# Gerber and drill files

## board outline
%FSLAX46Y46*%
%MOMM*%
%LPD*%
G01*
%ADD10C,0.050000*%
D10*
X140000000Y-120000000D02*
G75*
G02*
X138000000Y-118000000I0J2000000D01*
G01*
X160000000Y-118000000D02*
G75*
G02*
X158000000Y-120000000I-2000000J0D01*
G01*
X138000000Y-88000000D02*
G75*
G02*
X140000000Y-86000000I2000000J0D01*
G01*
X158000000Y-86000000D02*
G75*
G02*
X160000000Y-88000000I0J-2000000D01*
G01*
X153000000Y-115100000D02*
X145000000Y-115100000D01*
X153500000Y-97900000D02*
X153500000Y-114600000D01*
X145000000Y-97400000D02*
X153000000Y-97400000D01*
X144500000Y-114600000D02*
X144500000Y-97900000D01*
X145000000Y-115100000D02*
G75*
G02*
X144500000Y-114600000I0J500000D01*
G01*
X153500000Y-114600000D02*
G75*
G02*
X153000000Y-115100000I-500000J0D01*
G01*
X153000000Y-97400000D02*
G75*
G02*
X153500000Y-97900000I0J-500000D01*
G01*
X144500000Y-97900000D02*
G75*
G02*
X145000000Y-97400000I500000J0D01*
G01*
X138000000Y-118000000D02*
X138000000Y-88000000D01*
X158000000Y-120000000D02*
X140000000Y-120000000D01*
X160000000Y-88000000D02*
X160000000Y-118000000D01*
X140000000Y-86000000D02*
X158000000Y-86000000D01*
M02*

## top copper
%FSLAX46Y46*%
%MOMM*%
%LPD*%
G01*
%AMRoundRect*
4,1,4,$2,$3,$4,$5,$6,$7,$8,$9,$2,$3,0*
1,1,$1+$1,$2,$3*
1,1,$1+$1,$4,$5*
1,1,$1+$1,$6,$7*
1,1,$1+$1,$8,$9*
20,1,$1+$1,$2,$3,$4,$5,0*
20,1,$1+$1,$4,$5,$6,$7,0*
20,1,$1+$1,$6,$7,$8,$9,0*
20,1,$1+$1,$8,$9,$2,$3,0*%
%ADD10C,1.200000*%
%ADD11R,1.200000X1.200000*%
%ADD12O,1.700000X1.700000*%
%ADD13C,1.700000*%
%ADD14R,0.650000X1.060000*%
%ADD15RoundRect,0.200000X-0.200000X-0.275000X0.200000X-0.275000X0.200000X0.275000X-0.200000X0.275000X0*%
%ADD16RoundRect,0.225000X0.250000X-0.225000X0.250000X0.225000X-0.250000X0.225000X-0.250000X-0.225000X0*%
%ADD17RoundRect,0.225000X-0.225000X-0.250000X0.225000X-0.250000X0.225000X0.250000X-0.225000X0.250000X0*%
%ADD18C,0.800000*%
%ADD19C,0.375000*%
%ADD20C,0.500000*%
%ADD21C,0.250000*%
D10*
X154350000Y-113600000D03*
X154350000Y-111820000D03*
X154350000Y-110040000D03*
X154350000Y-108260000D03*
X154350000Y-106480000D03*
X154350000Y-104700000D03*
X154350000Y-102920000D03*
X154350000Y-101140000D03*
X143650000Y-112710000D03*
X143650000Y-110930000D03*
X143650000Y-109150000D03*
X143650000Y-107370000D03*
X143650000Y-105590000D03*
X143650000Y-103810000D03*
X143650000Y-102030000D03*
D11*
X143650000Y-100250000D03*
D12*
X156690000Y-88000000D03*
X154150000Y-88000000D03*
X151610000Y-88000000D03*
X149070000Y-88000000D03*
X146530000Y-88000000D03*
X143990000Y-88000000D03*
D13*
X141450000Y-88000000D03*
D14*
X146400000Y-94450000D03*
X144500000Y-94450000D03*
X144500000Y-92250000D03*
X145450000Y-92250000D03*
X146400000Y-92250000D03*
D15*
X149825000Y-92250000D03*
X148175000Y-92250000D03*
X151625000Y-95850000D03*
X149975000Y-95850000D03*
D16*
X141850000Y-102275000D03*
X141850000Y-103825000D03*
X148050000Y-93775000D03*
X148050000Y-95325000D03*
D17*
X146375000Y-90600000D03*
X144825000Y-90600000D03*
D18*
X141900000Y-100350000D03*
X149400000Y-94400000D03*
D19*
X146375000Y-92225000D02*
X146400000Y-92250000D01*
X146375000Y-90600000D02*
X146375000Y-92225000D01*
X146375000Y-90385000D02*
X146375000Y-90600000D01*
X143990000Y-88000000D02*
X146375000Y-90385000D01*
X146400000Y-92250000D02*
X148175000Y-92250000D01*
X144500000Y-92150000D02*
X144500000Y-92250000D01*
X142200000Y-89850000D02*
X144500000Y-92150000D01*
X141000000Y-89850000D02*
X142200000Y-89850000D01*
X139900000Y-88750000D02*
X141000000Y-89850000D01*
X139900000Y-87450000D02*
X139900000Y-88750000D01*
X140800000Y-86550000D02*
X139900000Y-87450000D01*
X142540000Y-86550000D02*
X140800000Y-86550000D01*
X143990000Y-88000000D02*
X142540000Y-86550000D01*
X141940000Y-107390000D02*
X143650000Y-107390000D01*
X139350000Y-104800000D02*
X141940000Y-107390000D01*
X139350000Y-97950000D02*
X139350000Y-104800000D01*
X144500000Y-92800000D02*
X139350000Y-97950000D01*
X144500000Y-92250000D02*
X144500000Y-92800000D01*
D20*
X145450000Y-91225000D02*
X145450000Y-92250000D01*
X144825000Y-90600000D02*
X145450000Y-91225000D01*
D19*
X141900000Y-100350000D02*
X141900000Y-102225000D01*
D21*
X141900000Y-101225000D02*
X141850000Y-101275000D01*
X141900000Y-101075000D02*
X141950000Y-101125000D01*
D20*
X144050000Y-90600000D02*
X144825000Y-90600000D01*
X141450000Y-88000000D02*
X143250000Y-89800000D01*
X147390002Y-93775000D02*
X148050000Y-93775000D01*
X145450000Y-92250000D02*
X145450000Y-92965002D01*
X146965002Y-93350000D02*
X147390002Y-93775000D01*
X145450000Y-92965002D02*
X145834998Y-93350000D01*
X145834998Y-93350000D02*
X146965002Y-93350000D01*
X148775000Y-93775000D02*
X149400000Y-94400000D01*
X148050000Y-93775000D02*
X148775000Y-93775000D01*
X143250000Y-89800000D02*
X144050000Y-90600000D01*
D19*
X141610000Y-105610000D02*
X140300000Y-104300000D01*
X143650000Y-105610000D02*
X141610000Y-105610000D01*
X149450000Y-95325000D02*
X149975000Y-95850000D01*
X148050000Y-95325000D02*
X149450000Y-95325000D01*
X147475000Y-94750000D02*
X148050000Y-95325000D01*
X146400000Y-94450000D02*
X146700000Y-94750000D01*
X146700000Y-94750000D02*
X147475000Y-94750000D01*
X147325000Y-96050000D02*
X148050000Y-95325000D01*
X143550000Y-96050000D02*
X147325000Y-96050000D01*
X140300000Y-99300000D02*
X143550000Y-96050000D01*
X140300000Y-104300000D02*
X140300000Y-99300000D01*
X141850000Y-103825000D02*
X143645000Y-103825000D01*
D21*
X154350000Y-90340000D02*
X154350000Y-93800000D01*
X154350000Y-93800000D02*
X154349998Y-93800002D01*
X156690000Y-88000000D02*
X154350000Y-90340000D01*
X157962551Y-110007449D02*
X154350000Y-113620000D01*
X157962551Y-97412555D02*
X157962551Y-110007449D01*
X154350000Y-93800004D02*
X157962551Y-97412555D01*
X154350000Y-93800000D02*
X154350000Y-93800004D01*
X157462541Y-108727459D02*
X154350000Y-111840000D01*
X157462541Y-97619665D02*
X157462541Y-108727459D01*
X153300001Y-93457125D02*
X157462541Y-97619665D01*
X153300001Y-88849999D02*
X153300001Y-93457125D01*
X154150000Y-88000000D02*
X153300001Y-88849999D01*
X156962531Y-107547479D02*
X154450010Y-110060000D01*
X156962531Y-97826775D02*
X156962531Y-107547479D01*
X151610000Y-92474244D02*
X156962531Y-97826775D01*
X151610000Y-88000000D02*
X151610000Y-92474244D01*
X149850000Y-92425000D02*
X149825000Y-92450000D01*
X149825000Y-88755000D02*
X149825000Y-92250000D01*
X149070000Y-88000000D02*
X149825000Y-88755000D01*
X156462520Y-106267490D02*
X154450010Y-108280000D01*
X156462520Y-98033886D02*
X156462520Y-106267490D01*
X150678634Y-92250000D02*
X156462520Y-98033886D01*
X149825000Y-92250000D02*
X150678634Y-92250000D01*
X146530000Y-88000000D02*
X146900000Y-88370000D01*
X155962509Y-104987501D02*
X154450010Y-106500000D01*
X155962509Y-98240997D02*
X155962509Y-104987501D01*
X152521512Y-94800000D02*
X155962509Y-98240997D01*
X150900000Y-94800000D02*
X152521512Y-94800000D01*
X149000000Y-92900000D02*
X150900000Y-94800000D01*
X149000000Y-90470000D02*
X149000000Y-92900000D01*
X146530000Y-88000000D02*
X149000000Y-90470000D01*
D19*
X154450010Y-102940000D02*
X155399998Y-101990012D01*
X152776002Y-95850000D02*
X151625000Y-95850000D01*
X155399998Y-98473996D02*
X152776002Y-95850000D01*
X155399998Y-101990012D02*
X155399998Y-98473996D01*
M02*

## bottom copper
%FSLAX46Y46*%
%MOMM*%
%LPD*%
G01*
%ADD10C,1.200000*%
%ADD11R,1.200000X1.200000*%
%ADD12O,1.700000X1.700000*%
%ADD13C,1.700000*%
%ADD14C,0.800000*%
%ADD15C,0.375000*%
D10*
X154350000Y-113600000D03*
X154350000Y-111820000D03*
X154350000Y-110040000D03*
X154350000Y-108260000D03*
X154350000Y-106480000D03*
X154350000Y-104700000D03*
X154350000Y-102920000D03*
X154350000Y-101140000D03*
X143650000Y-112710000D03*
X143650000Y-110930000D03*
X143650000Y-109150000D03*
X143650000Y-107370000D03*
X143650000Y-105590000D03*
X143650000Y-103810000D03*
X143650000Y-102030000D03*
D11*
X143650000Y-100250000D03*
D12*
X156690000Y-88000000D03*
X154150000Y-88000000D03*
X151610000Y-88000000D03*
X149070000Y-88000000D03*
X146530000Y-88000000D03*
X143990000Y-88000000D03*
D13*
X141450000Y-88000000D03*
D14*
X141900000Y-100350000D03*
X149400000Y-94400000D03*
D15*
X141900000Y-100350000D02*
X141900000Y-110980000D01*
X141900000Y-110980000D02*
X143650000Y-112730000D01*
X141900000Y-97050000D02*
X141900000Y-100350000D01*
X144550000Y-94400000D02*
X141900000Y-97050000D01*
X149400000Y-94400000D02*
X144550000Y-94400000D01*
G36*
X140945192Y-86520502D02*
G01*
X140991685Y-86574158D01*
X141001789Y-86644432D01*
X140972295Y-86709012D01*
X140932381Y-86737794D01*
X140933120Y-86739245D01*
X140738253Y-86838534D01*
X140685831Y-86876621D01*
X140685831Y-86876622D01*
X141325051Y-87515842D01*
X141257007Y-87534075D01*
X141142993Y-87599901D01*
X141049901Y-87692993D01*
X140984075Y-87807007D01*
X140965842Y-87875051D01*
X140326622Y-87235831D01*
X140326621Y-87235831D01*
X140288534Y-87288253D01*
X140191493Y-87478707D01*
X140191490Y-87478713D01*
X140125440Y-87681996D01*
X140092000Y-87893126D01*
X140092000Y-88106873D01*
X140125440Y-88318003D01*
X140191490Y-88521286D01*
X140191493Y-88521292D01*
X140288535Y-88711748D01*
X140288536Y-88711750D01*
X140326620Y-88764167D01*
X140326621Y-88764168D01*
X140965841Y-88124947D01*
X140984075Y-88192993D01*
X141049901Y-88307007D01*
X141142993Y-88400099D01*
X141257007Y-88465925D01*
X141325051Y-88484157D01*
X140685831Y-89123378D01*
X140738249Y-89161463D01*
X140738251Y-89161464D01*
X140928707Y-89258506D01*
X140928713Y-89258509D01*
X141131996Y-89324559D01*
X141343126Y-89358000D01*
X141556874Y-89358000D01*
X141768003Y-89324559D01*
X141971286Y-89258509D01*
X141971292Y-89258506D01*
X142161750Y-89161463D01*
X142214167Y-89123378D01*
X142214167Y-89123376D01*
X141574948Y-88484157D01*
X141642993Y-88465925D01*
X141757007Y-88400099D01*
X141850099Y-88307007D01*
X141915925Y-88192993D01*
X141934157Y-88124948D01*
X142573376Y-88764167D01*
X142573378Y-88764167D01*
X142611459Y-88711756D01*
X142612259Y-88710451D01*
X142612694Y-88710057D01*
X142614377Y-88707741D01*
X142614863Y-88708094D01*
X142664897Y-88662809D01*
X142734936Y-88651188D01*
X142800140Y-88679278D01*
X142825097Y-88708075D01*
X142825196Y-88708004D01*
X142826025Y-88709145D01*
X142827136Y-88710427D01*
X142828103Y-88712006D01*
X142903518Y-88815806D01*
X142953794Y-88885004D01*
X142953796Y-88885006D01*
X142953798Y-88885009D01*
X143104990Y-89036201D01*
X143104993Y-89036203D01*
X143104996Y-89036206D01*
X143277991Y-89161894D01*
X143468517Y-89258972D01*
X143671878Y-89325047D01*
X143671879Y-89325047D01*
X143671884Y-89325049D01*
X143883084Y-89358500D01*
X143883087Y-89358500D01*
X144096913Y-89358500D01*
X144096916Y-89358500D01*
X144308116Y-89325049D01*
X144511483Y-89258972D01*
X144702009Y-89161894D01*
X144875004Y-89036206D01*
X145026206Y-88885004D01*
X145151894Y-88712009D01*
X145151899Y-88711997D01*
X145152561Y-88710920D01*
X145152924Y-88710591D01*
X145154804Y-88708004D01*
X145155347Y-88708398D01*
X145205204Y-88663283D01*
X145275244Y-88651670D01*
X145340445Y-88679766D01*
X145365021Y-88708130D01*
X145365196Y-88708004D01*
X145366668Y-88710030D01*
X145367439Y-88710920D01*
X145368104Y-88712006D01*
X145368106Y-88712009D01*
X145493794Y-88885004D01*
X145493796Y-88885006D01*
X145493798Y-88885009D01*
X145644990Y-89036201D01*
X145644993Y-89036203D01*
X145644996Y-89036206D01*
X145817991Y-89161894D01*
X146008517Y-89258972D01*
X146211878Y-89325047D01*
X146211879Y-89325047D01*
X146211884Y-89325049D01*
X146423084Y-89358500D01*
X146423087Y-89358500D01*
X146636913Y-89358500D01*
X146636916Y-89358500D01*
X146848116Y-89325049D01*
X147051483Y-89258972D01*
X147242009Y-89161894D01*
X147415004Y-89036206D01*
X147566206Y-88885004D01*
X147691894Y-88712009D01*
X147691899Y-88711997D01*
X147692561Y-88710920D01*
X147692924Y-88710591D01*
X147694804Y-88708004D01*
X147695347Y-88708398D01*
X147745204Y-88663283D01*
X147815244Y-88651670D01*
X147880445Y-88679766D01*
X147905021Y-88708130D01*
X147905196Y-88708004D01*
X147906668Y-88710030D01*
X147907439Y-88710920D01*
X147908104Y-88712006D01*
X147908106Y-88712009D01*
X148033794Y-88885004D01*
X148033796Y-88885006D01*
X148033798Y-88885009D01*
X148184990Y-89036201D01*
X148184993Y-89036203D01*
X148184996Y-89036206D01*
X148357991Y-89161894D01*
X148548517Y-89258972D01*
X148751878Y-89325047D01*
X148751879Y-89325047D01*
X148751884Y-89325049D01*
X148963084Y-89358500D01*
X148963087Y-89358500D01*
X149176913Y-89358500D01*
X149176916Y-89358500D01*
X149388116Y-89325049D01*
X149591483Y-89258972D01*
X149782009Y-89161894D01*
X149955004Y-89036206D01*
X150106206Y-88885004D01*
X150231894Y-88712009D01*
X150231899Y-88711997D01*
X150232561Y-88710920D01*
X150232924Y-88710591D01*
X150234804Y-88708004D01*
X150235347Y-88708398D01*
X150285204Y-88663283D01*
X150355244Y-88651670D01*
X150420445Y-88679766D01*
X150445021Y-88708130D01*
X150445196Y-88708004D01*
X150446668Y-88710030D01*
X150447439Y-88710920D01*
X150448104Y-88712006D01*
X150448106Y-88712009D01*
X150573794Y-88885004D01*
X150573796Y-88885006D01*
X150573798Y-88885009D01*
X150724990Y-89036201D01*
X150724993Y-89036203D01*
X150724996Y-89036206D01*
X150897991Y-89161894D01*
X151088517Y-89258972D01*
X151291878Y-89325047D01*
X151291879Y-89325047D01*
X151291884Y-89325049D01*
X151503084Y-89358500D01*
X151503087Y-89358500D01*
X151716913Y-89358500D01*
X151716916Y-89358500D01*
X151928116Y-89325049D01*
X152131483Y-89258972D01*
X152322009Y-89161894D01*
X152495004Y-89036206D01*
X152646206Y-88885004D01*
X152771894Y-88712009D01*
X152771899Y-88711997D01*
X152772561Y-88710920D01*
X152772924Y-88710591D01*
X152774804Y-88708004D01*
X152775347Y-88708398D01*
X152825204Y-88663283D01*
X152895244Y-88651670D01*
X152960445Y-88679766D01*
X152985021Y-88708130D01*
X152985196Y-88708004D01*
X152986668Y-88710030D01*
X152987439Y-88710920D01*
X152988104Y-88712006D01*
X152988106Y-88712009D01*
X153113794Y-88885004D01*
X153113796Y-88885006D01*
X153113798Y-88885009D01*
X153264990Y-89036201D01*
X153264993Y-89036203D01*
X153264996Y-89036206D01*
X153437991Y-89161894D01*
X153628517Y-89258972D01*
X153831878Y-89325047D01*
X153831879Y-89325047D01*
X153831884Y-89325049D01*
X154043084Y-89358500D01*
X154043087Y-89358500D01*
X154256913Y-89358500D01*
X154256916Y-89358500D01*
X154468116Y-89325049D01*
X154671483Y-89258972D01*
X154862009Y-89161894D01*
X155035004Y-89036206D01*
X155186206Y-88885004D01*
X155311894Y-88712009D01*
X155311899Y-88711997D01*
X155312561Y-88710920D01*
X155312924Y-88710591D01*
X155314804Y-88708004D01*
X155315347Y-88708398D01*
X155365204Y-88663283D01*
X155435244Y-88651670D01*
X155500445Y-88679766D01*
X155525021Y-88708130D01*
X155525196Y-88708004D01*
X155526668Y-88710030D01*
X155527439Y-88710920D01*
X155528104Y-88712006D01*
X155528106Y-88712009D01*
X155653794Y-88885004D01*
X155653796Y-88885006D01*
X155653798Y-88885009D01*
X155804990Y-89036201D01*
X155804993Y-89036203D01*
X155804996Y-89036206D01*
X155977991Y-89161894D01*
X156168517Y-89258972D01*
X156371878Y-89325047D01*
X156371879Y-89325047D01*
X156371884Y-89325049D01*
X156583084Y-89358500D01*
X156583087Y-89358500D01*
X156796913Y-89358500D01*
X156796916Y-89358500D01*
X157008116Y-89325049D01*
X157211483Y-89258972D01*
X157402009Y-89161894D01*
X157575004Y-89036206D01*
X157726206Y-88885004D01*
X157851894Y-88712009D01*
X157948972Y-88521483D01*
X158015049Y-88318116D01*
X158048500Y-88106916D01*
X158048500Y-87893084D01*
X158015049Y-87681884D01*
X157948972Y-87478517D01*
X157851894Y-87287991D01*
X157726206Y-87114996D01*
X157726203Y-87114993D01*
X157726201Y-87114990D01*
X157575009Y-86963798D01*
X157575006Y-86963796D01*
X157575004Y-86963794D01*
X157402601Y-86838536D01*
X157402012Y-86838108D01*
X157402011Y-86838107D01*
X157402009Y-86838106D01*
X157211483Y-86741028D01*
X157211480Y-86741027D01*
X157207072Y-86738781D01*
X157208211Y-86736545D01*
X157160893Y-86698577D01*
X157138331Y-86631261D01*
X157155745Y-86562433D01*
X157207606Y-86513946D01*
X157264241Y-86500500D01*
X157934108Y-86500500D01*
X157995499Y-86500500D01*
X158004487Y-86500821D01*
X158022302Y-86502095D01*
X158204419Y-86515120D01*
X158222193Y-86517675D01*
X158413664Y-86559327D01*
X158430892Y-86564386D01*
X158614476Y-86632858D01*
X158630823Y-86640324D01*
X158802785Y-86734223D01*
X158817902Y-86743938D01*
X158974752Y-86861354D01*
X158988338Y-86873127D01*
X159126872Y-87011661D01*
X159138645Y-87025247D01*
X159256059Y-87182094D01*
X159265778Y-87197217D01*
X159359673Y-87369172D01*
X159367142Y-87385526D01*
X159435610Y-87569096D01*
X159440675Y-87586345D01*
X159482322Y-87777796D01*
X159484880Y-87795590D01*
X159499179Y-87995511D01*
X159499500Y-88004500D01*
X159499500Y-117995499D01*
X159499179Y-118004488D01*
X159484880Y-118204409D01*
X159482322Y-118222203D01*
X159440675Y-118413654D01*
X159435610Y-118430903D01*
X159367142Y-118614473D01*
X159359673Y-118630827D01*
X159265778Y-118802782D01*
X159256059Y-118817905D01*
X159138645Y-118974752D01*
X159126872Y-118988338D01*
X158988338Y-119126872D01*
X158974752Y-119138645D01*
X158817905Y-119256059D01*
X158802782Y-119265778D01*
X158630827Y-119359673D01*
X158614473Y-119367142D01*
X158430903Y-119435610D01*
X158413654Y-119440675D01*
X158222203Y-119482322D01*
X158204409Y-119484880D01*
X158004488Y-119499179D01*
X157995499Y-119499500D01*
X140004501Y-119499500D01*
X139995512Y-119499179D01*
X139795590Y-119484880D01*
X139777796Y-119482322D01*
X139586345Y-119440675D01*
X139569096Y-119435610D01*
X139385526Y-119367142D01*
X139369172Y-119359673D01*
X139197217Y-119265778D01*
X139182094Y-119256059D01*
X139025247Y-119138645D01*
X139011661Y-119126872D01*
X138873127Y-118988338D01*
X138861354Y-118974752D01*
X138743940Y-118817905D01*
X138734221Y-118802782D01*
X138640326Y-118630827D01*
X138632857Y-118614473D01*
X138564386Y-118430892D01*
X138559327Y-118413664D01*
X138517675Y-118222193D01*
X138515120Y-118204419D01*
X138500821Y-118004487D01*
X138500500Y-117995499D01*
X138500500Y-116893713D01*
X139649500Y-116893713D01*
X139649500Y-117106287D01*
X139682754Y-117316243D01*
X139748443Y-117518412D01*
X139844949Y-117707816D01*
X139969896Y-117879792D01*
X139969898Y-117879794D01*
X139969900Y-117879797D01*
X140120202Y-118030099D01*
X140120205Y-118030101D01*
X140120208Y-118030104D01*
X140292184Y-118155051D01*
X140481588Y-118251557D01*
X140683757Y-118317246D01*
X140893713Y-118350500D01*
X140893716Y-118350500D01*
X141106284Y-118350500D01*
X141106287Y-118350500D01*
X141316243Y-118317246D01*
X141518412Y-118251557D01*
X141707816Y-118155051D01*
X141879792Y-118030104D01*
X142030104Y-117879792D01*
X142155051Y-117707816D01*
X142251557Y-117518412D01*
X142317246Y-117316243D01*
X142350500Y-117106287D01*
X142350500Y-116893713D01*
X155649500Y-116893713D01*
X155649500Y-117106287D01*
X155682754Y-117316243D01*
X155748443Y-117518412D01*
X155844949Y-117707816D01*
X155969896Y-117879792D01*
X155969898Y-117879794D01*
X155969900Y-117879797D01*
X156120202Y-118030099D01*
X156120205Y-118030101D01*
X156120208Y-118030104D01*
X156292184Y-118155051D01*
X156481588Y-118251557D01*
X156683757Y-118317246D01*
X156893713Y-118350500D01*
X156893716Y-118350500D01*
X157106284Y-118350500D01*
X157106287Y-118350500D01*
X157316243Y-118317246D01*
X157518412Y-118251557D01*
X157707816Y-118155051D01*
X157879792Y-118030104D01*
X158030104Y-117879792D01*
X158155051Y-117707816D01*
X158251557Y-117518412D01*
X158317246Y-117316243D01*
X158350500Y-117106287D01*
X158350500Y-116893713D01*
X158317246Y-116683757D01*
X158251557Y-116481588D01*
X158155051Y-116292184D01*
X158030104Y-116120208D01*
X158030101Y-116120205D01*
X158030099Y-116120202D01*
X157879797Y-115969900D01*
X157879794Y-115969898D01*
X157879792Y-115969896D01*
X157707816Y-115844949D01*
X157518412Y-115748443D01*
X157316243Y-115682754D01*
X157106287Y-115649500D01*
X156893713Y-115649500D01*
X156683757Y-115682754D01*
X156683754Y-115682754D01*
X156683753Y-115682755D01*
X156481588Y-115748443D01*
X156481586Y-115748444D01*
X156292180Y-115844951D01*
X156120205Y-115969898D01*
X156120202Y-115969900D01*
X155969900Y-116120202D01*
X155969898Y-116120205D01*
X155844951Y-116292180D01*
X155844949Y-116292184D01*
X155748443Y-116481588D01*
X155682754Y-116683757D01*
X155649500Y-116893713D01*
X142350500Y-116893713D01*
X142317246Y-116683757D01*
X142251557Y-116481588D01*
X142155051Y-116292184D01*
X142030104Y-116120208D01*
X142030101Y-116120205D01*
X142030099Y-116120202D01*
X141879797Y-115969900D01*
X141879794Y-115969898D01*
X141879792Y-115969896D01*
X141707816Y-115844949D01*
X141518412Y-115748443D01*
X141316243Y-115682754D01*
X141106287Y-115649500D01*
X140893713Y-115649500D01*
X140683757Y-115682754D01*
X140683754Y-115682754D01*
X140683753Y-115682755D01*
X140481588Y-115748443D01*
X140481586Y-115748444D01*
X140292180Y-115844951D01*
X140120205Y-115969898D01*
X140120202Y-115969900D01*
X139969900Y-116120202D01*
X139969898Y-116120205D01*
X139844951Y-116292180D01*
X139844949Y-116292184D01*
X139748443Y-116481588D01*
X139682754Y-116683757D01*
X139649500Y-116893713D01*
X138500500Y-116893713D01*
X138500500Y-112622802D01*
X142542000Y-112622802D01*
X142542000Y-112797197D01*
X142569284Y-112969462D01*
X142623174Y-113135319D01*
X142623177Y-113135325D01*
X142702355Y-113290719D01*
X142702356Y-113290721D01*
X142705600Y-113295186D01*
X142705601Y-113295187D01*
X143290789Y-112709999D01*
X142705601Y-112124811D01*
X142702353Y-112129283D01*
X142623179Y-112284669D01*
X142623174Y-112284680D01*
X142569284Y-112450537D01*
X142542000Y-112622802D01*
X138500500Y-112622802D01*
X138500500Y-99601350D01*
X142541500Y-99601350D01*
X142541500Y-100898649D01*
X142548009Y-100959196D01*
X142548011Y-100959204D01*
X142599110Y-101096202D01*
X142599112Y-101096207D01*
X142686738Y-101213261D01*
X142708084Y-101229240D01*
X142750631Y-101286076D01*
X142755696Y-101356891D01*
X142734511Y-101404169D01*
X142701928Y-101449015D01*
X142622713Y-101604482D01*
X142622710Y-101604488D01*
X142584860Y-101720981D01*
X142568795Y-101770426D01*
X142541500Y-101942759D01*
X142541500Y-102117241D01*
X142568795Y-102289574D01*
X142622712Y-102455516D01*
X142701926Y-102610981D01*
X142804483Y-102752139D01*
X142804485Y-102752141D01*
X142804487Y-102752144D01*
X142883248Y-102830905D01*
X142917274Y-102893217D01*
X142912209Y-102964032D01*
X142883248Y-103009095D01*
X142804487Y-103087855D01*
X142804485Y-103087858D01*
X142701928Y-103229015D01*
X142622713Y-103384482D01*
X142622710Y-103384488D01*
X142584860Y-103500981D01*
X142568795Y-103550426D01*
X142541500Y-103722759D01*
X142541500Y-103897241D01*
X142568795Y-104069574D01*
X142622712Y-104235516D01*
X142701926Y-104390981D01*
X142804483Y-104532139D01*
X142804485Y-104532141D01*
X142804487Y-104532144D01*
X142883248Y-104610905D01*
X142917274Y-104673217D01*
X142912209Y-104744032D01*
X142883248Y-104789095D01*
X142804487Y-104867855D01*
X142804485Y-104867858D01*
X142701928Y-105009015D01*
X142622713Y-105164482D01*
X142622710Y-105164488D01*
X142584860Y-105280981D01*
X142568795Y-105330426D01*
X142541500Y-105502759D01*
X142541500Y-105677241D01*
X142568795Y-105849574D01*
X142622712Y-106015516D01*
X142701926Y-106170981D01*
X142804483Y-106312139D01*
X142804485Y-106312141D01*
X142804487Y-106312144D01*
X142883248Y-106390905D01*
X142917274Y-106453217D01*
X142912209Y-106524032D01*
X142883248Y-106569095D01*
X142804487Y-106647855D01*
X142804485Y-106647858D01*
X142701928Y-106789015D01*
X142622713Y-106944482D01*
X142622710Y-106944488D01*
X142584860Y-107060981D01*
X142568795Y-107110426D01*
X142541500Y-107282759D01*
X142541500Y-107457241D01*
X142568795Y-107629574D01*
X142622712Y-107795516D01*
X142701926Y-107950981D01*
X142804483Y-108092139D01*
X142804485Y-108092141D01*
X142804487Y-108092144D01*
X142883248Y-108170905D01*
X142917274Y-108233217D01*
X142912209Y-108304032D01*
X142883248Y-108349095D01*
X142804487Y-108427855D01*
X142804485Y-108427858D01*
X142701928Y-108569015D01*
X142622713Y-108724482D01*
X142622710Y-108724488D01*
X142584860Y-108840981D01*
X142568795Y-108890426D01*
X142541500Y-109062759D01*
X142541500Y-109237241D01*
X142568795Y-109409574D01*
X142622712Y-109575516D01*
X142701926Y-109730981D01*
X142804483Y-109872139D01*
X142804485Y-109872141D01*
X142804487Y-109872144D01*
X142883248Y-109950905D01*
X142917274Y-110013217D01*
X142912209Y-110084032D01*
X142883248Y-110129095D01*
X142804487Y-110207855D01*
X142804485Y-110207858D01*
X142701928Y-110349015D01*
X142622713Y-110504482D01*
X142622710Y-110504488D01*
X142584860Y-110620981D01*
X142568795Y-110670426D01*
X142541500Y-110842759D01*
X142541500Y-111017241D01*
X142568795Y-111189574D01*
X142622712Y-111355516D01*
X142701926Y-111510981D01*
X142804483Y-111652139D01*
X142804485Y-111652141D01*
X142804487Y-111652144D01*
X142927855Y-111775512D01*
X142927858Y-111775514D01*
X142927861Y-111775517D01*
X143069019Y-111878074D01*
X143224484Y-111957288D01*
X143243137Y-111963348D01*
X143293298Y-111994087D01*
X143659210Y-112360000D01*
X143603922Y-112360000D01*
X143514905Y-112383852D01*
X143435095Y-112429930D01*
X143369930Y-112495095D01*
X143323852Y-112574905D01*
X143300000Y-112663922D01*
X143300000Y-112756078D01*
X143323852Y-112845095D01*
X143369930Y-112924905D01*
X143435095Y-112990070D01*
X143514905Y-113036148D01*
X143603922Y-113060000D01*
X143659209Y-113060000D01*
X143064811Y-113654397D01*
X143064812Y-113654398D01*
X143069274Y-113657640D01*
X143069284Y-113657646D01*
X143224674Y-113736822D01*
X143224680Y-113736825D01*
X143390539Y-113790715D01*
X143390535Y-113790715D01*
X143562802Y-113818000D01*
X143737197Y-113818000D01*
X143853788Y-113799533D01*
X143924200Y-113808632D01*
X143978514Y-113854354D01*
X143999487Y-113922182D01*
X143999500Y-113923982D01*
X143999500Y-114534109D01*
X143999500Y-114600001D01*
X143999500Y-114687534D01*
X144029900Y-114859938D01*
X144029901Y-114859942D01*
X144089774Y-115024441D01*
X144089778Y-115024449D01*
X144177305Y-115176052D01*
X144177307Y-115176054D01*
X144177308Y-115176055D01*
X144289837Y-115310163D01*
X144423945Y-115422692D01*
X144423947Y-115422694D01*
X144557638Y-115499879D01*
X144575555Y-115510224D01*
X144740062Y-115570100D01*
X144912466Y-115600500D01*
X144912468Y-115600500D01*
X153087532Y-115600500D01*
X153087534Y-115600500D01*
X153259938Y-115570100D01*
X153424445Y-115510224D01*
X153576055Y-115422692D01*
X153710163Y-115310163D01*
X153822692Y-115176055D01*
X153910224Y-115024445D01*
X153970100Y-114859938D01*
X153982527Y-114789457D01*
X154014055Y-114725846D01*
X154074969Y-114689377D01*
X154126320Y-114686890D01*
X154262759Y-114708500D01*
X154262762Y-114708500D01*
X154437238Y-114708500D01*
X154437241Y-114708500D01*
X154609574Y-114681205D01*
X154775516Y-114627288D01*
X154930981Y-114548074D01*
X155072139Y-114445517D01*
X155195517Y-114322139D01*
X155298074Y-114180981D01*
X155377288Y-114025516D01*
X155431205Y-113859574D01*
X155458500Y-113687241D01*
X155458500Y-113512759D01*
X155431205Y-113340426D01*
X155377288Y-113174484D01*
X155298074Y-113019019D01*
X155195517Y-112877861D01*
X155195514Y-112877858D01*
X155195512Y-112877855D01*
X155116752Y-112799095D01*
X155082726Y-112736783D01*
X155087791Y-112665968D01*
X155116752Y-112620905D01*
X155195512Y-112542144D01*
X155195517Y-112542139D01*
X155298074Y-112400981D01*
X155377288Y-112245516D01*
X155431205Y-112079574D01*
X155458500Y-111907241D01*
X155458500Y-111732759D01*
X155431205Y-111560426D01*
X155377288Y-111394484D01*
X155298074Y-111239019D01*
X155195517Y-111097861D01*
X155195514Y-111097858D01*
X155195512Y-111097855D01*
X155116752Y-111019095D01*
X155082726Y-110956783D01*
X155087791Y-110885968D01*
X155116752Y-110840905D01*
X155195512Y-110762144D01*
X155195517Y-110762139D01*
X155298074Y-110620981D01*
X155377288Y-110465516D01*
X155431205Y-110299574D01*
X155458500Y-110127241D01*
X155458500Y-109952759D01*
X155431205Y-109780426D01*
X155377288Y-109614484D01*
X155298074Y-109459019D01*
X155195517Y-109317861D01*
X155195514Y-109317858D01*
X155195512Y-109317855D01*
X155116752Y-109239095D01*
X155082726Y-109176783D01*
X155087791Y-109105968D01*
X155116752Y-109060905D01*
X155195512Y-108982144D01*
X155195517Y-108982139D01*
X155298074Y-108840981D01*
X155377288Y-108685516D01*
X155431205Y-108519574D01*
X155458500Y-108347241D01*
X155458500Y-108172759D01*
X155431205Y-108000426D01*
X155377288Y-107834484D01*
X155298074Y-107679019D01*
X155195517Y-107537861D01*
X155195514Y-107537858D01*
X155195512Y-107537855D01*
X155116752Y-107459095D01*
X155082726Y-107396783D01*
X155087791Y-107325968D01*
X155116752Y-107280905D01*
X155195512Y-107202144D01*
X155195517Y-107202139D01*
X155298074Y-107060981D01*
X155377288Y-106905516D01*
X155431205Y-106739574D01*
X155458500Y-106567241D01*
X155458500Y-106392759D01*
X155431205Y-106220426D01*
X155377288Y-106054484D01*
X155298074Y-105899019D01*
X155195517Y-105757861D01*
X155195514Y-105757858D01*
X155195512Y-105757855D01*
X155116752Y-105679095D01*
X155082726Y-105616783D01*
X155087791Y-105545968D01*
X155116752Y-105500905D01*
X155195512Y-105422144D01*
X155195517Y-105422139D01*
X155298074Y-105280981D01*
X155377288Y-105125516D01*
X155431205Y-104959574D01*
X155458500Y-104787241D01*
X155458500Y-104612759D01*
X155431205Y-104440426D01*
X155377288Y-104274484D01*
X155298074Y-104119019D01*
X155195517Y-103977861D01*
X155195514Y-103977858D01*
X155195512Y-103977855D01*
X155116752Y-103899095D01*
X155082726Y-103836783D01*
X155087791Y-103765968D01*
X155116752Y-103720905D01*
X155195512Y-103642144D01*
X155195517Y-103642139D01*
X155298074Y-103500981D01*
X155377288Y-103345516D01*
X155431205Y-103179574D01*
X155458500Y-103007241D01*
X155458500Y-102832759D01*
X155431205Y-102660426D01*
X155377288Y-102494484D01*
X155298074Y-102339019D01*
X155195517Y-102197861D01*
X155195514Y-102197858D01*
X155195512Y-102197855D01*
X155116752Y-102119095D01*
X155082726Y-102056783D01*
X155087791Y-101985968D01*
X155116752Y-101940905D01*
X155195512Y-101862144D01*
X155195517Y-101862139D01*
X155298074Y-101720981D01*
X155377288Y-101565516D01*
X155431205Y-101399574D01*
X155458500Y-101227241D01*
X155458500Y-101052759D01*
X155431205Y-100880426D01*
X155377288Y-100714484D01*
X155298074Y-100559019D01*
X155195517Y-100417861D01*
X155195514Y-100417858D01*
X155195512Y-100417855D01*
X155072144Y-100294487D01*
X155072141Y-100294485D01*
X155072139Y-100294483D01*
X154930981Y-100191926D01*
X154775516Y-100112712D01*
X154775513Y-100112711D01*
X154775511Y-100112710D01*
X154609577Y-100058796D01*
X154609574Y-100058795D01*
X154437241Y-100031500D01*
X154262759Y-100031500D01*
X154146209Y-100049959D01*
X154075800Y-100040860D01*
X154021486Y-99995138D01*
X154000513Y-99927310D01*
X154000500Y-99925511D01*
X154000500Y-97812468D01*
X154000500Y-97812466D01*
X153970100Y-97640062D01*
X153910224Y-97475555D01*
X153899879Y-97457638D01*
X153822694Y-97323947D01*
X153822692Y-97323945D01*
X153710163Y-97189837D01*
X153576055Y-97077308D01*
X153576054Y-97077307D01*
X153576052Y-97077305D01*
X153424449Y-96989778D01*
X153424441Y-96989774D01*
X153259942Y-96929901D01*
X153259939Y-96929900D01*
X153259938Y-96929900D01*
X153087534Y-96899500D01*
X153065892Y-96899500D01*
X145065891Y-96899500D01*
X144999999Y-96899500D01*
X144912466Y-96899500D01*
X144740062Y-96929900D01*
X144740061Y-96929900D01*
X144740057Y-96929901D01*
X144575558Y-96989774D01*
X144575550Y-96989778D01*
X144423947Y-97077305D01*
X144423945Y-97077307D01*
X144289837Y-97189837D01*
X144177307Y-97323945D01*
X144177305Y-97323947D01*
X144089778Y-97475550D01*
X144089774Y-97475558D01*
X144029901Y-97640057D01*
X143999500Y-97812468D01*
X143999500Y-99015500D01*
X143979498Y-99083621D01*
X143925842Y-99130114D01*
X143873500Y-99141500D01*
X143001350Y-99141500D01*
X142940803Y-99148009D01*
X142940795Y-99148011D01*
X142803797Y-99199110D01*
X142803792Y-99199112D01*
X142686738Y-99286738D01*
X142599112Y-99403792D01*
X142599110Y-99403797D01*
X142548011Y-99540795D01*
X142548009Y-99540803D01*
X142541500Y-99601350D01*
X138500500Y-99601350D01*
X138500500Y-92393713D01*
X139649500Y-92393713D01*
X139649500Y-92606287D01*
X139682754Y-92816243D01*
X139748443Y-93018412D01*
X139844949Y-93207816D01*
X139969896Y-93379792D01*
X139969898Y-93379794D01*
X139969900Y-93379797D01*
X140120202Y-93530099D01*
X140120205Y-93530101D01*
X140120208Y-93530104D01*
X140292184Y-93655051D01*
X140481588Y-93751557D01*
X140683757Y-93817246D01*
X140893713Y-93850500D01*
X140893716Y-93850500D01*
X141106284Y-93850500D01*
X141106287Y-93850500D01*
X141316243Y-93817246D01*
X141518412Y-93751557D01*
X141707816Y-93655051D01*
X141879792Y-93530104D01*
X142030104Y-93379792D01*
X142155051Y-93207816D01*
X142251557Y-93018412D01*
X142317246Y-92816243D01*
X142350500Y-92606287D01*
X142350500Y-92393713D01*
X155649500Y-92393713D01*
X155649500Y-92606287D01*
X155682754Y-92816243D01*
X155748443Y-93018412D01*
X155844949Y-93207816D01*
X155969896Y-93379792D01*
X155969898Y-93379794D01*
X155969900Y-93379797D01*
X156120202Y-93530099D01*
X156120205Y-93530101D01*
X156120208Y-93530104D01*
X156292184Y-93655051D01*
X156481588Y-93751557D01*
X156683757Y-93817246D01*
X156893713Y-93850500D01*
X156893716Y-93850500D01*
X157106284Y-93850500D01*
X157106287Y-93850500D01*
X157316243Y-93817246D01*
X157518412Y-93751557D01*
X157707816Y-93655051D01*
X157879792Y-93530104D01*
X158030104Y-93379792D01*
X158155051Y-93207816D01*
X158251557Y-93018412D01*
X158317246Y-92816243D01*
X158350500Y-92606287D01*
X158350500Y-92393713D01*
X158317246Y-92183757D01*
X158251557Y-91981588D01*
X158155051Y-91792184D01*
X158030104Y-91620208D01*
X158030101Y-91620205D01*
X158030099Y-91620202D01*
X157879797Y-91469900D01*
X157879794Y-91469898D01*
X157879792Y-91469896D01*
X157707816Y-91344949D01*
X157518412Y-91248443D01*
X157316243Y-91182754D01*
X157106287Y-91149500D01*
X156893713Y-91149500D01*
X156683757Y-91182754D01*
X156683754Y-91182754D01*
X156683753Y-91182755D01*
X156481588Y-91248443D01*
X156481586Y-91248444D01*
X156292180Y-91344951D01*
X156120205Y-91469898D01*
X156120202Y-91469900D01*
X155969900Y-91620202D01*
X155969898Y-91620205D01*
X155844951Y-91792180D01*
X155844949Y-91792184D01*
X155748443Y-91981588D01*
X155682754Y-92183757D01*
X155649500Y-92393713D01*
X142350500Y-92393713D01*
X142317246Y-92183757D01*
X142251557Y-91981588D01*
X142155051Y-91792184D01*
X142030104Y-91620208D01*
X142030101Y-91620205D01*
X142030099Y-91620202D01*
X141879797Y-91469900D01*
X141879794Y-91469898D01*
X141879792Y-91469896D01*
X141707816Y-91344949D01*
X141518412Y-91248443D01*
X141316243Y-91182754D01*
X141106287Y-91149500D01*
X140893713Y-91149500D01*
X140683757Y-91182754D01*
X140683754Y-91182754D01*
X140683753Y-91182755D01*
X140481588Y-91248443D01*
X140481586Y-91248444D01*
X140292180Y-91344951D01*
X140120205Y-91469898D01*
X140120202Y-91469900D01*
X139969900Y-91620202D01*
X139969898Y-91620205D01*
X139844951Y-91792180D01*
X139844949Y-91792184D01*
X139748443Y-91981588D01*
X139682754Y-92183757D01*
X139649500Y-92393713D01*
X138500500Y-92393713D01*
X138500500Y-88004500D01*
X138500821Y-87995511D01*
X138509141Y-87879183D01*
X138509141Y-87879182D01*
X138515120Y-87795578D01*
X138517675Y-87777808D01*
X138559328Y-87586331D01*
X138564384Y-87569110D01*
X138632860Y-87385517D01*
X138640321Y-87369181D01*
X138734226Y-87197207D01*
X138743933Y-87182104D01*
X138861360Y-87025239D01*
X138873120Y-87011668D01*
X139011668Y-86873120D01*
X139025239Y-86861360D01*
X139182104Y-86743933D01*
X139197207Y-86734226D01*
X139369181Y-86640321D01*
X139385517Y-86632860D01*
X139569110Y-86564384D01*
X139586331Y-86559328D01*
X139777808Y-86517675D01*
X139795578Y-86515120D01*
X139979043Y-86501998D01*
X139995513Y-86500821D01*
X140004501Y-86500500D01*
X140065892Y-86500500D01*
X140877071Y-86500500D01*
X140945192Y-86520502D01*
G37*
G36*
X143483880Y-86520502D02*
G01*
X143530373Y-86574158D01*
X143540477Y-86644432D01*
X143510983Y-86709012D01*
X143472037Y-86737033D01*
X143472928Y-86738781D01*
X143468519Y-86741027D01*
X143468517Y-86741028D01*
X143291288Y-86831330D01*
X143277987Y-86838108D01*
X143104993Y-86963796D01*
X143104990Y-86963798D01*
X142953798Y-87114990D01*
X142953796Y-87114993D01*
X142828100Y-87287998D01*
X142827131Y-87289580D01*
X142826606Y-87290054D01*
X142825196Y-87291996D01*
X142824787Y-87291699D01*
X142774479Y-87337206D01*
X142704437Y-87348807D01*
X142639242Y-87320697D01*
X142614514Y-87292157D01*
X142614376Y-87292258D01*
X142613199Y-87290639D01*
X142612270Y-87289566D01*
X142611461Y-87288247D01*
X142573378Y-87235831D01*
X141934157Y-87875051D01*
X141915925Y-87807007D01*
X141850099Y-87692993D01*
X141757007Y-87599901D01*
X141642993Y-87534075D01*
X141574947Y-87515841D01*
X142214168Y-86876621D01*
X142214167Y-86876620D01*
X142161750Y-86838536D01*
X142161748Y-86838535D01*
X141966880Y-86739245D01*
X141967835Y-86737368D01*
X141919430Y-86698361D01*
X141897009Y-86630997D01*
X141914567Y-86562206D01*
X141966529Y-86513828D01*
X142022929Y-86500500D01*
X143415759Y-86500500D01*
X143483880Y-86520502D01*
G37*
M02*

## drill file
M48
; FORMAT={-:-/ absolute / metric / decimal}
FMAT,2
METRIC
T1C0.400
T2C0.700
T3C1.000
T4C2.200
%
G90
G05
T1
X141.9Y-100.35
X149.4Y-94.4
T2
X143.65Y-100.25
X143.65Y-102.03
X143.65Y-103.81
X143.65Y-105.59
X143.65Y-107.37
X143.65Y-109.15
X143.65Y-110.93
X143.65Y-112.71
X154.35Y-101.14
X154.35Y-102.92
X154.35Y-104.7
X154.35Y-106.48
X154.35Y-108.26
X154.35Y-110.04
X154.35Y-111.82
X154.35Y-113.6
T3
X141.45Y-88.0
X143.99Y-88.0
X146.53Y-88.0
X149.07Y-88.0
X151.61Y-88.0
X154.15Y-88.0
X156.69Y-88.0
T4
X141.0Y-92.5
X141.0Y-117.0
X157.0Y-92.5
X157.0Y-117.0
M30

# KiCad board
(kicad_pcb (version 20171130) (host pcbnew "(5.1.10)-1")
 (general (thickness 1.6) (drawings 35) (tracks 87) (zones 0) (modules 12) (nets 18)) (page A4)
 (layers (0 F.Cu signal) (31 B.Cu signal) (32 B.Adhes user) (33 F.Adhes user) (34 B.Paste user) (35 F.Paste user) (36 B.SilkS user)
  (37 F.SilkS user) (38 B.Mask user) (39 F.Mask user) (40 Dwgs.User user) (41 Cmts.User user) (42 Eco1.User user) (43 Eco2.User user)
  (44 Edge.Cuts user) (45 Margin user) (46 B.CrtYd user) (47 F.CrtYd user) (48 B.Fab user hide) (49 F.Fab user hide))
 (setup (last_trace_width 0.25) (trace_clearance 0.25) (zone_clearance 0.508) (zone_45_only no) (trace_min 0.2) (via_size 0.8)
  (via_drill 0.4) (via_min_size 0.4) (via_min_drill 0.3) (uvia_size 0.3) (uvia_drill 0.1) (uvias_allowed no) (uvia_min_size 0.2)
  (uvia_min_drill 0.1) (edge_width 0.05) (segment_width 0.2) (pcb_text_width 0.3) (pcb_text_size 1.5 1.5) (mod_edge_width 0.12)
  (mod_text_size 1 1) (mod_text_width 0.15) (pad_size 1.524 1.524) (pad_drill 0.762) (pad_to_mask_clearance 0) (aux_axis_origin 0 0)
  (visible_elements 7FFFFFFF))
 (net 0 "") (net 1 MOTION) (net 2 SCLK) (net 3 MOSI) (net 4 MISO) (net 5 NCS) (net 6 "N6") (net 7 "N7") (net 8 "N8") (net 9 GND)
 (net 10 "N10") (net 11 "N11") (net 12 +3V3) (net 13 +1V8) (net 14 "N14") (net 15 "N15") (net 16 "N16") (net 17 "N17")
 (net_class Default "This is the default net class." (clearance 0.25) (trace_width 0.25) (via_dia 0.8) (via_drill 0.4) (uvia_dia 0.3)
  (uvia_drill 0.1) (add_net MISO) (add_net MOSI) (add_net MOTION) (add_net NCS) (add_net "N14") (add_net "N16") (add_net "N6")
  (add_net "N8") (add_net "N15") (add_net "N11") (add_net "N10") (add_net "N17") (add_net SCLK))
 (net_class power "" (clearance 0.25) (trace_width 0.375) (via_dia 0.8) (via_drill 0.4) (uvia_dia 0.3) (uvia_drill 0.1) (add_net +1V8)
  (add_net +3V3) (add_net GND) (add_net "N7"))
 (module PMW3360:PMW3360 (layer F.Cu) (at 143.65 100.25)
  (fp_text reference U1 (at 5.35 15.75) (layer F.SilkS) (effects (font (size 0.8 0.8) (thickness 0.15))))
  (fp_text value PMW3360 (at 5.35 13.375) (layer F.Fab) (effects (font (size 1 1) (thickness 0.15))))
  (pad 9 thru_hole circle (at 10.7 13.35) (size 1.2 1.2) (drill 0.7) (layers *.Cu *.Mask) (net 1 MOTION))
  (pad 10 thru_hole circle (at 10.7 11.57) (size 1.2 1.2) (drill 0.7) (layers *.Cu *.Mask) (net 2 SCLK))
  (pad 11 thru_hole circle (at 10.7 9.79) (size 1.2 1.2) (drill 0.7) (layers *.Cu *.Mask) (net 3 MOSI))
  (pad 12 thru_hole circle (at 10.7 8.01) (size 1.2 1.2) (drill 0.7) (layers *.Cu *.Mask) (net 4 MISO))
  (pad 13 thru_hole circle (at 10.7 6.23) (size 1.2 1.2) (drill 0.7) (layers *.Cu *.Mask) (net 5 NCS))
  (pad 14 thru_hole circle (at 10.7 4.45) (size 1.2 1.2) (drill 0.7) (layers *.Cu *.Mask) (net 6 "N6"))
  (pad 15 thru_hole circle (at 10.7 2.67) (size 1.2 1.2) (drill 0.7) (layers *.Cu *.Mask) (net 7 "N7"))
  (pad 16 thru_hole circle (at 10.7 0.89) (size 1.2 1.2) (drill 0.7) (layers *.Cu *.Mask) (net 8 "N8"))
  (pad 8 thru_hole circle (at 0 12.46) (size 1.2 1.2) (drill 0.7) (layers *.Cu *.Mask) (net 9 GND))
  (pad 7 thru_hole circle (at 0 10.68) (size 1.2 1.2) (drill 0.7) (layers *.Cu *.Mask) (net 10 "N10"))
  (pad 6 thru_hole circle (at 0 8.9) (size 1.2 1.2) (drill 0.7) (layers *.Cu *.Mask) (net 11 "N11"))
  (pad 5 thru_hole circle (at 0 7.12) (size 1.2 1.2) (drill 0.7) (layers *.Cu *.Mask) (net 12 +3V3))
  (pad 4 thru_hole circle (at 0 5.34) (size 1.2 1.2) (drill 0.7) (layers *.Cu *.Mask) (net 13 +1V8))
  (pad 3 thru_hole circle (at 0 3.56) (size 1.2 1.2) (drill 0.7) (layers *.Cu *.Mask) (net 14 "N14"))
  (pad 2 thru_hole circle (at 0 1.78) (size 1.2 1.2) (drill 0.7) (layers *.Cu *.Mask) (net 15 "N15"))
  (pad 1 thru_hole rect (at 0 0) (size 1.2 1.2) (drill 0.7) (layers *.Cu *.Mask) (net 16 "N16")))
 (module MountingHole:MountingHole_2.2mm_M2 (layer F.Cu) (at 141 92.5)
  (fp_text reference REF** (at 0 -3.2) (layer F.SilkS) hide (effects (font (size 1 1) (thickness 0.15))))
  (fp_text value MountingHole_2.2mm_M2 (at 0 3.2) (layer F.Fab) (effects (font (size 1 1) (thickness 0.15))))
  (pad 1 np_thru_hole circle (at 0 0) (size 2.2 2.2) (drill 2.2) (layers *.Cu *.Mask)))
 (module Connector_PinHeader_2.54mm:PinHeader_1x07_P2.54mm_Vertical (layer F.Cu) (at 141.45 88 90)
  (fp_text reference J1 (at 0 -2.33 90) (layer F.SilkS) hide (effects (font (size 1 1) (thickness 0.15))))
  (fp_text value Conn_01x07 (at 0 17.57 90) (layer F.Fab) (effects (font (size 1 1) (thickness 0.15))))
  (pad 7 thru_hole oval (at 0 15.24 90) (size 1.7 1.7) (drill 1) (layers *.Cu *.Mask) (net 1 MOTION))
  (pad 6 thru_hole oval (at 0 12.7 90) (size 1.7 1.7) (drill 1) (layers *.Cu *.Mask) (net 2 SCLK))
  (pad 5 thru_hole oval (at 0 10.16 90) (size 1.7 1.7) (drill 1) (layers *.Cu *.Mask) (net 3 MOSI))
  (pad 4 thru_hole oval (at 0 7.62 90) (size 1.7 1.7) (drill 1) (layers *.Cu *.Mask) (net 4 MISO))
  (pad 3 thru_hole oval (at 0 5.08 90) (size 1.7 1.7) (drill 1) (layers *.Cu *.Mask) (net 5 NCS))
  (pad 2 thru_hole oval (at 0 2.54 90) (size 1.7 1.7) (drill 1) (layers *.Cu *.Mask) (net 12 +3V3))
  (pad 1 thru_hole circle (at 0 0 90) (size 1.7 1.7) (drill 1) (layers *.Cu *.Mask) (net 9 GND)))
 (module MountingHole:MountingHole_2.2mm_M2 (layer F.Cu) (at 157 117)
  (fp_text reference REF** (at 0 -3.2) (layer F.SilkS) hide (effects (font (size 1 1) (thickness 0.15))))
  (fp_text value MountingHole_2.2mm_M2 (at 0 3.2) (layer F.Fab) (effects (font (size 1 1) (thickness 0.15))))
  (pad 1 np_thru_hole circle (at 0 0) (size 2.2 2.2) (drill 2.2) (layers *.Cu *.Mask)))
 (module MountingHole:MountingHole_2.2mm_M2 (layer F.Cu) (at 141 117)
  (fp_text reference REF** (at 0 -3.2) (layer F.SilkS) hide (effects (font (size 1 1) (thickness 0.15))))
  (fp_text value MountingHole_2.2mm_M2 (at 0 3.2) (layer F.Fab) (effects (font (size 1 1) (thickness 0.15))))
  (pad 1 np_thru_hole circle (at 0 0) (size 2.2 2.2) (drill 2.2) (layers *.Cu *.Mask)))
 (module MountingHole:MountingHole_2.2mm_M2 (layer F.Cu) (at 157 92.5)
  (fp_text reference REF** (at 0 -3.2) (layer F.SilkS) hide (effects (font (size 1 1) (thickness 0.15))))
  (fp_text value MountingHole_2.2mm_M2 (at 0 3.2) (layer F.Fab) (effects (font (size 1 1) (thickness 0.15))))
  (pad 1 np_thru_hole circle (at 0 0) (size 2.2 2.2) (drill 2.2) (layers *.Cu *.Mask)))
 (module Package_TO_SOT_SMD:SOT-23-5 (layer F.Cu) (at 145.45 93.35 270)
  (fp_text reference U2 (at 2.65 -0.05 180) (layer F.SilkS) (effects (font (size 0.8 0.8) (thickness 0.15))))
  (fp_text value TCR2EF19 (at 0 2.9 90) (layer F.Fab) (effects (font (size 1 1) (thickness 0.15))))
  (pad 5 smd rect (at 1.1 -0.95 270) (size 1.06 0.65) (layers F.Cu F.Paste F.Mask) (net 13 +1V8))
  (pad 4 smd rect (at 1.1 0.95 270) (size 1.06 0.65) (layers F.Cu F.Paste F.Mask) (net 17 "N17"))
  (pad 3 smd rect (at -1.1 0.95 270) (size 1.06 0.65) (layers F.Cu F.Paste F.Mask) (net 12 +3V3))
  (pad 2 smd rect (at -1.1 0 270) (size 1.06 0.65) (layers F.Cu F.Paste F.Mask) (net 9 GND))
  (pad 1 smd rect (at -1.1 -0.95 270) (size 1.06 0.65) (layers F.Cu F.Paste F.Mask) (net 12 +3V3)))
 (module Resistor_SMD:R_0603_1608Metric (layer F.Cu) (at 149 92.25)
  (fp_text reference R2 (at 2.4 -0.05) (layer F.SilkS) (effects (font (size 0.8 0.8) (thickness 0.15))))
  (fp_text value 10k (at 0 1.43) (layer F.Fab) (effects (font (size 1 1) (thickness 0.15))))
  (pad 2 smd roundrect (at 0.825 0) (size 0.8 0.95) (layers F.Cu F.Paste F.Mask) (roundrect_rratio 0.25) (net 4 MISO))
  (pad 1 smd roundrect (at -0.825 0) (size 0.8 0.95) (layers F.Cu F.Paste F.Mask) (roundrect_rratio 0.25) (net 12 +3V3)))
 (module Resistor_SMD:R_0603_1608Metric (layer F.Cu) (at 150.8 95.85)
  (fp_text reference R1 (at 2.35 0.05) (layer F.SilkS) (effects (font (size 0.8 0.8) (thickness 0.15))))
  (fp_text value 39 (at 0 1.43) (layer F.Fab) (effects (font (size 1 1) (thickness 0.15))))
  (pad 2 smd roundrect (at 0.825 0) (size 0.8 0.95) (layers F.Cu F.Paste F.Mask) (roundrect_rratio 0.25) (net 7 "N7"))
  (pad 1 smd roundrect (at -0.825 0) (size 0.8 0.95) (layers F.Cu F.Paste F.Mask) (roundrect_rratio 0.25) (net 13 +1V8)))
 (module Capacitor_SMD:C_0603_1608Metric (layer F.Cu) (at 141.85 103.05 90)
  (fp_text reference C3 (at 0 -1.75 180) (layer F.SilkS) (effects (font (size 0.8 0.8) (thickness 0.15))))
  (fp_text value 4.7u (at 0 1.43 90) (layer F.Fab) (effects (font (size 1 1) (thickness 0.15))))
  (pad 2 smd roundrect (at 0.775 0 90) (size 0.9 0.95) (layers F.Cu F.Paste F.Mask) (roundrect_rratio 0.25) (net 9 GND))
  (pad 1 smd roundrect (at -0.775 0 90) (size 0.9 0.95) (layers F.Cu F.Paste F.Mask) (roundrect_rratio 0.25) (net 14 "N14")))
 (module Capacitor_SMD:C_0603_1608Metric (layer F.Cu) (at 148.05 94.55 90)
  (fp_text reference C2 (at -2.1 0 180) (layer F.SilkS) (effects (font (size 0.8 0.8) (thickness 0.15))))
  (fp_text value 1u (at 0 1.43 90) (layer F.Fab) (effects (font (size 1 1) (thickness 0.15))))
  (pad 2 smd roundrect (at 0.775 0 90) (size 0.9 0.95) (layers F.Cu F.Paste F.Mask) (roundrect_rratio 0.25) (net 9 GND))
  (pad 1 smd roundrect (at -0.775 0 90) (size 0.9 0.95) (layers F.Cu F.Paste F.Mask) (roundrect_rratio 0.25) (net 13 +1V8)))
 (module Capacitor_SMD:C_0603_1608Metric (layer F.Cu) (at 145.6 90.6)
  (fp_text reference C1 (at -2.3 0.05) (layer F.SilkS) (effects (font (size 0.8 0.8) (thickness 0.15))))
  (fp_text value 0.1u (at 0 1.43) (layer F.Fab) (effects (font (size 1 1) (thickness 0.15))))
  (pad 2 smd roundrect (at 0.775 0) (size 0.9 0.95) (layers F.Cu F.Paste F.Mask) (roundrect_rratio 0.25) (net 12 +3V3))
  (pad 1 smd roundrect (at -0.775 0) (size 0.9 0.95) (layers F.Cu F.Paste F.Mask) (roundrect_rratio 0.25) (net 9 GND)))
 (gr_arc (start 140 118) (end 138 118) (angle -90) (layer Edge.Cuts) (width 0.05))
 (gr_arc (start 158 118) (end 158 120) (angle -90) (layer Edge.Cuts) (width 0.05))
 (gr_arc (start 140 88) (end 140 86) (angle -90) (layer Edge.Cuts) (width 0.05))
 (gr_arc (start 158 88) (end 160 88) (angle -90) (layer Edge.Cuts) (width 0.05))
 (gr_line (start 153 115.1) (end 145 115.1) (layer Edge.Cuts) (width 0.05))
 (gr_line (start 153.5 97.9) (end 153.5 114.6) (layer Edge.Cuts) (width 0.05))
 (gr_line (start 145 97.4) (end 153 97.4) (layer Edge.Cuts) (width 0.05))
 (gr_line (start 144.5 114.6) (end 144.5 97.9) (layer Edge.Cuts) (width 0.05))
 (gr_arc (start 145 114.6) (end 144.5 114.6) (angle -90) (layer Edge.Cuts) (width 0.05))
 (gr_arc (start 153 114.6) (end 153 115.1) (angle -90) (layer Edge.Cuts) (width 0.05))
 (gr_arc (start 153 97.9) (end 153.5 97.9) (angle -90) (layer Edge.Cuts) (width 0.05))
 (gr_arc (start 145 97.9) (end 145 97.4) (angle -90) (layer Edge.Cuts) (width 0.05))
 (gr_line (start 138 118) (end 138 88) (layer Edge.Cuts) (width 0.05))
 (gr_line (start 158 120) (end 140 120) (layer Edge.Cuts) (width 0.05))
 (gr_line (start 160 88) (end 160 118) (layer Edge.Cuts) (width 0.05))
 (gr_line (start 140 86) (end 158 86) (layer Edge.Cuts) (width 0.05))
 (segment (start 146.375 92.225) (end 146.4 92.25) (width 0.375) (layer F.Cu) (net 12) (status 30))
 (segment (start 146.375 90.6) (end 146.375 92.225) (width 0.375) (layer F.Cu) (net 12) (status 30))
 (segment (start 146.375 90.385) (end 146.375 90.6) (width 0.375) (layer F.Cu) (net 12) (status 30))
 (segment (start 143.99 88) (end 146.375 90.385) (width 0.375) (layer F.Cu) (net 12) (status 30))
 (segment (start 146.4 92.25) (end 148.175 92.25) (width 0.375) (layer F.Cu) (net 12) (status 30))
 (segment (start 144.5 92.15) (end 144.5 92.25) (width 0.375) (layer F.Cu) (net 12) (status 30))
 (segment (start 142.2 89.85) (end 144.5 92.15) (width 0.375) (layer F.Cu) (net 12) (status 20))
 (segment (start 141 89.85) (end 142.2 89.85) (width 0.375) (layer F.Cu) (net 12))
 (segment (start 139.9 88.75) (end 141 89.85) (width 0.375) (layer F.Cu) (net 12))
 (segment (start 139.9 87.45) (end 139.9 88.75) (width 0.375) (layer F.Cu) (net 12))
 (segment (start 140.8 86.55) (end 139.9 87.45) (width 0.375) (layer F.Cu) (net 12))
 (segment (start 142.54 86.55) (end 140.8 86.55) (width 0.375) (layer F.Cu) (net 12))
 (segment (start 143.99 88) (end 142.54 86.55) (width 0.375) (layer F.Cu) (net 12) (status 10))
 (segment (start 141.94 107.39) (end 143.65 107.39) (width 0.375) (layer F.Cu) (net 12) (status 20))
 (segment (start 139.35 104.8) (end 141.94 107.39) (width 0.375) (layer F.Cu) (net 12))
 (segment (start 139.35 97.95) (end 139.35 104.8) (width 0.375) (layer F.Cu) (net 12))
 (segment (start 144.5 92.8) (end 139.35 97.95) (width 0.375) (layer F.Cu) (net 12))
 (segment (start 144.5 92.25) (end 144.5 92.8) (width 0.375) (layer F.Cu) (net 12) (status 10))
 (segment (start 145.45 91.225) (end 145.45 92.25) (width 0.5) (layer F.Cu) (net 9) (status 20))
 (segment (start 144.825 90.6) (end 145.45 91.225) (width 0.5) (layer F.Cu) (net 9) (status 10))
 (via (at 141.9 100.35) (size 0.8) (drill 0.4) (layers F.Cu B.Cu) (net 9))
 (segment (start 141.9 100.35) (end 141.9 102.225) (width 0.375) (layer F.Cu) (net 9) (status 20))
 (segment (start 141.9 101.225) (end 141.85 101.275) (width 0.25) (layer F.Cu) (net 9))
 (segment (start 141.9 101.075) (end 141.95 101.125) (width 0.25) (layer F.Cu) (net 9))
 (segment (start 141.9 100.35) (end 141.9 110.98) (width 0.375) (layer B.Cu) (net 9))
 (segment (start 144.05 90.6) (end 144.825 90.6) (width 0.5) (layer F.Cu) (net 9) (status 20))
 (segment (start 141.45 88) (end 143.25 89.8) (width 0.5) (layer F.Cu) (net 9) (status 10))
 (segment (start 147.390002 93.775) (end 148.05 93.775) (width 0.5) (layer F.Cu) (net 9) (status 20))
 (segment (start 145.45 92.25) (end 145.45 92.965002) (width 0.5) (layer F.Cu) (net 9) (status 10))
 (segment (start 146.965002 93.35) (end 147.390002 93.775) (width 0.5) (layer F.Cu) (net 9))
 (segment (start 145.45 92.965002) (end 145.834998 93.35) (width 0.5) (layer F.Cu) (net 9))
 (segment (start 145.834998 93.35) (end 146.965002 93.35) (width 0.5) (layer F.Cu) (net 9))
 (via (at 149.4 94.4) (size 0.8) (drill 0.4) (layers F.Cu B.Cu) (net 9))
 (segment (start 148.775 93.775) (end 149.4 94.4) (width 0.5) (layer F.Cu) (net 9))
 (segment (start 148.05 93.775) (end 148.775 93.775) (width 0.5) (layer F.Cu) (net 9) (status 10))
 (segment (start 141.9 110.98) (end 143.65 112.73) (width 0.375) (layer B.Cu) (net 9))
 (segment (start 143.25 89.8) (end 144.05 90.6) (width 0.5) (layer F.Cu) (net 9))
 (segment (start 141.9 97.05) (end 141.9 100.35) (width 0.375) (layer B.Cu) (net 9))
 (segment (start 144.55 94.4) (end 141.9 97.05) (width 0.375) (layer B.Cu) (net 9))
 (segment (start 149.4 94.4) (end 144.55 94.4) (width 0.375) (layer B.Cu) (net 9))
 (segment (start 141.61 105.61) (end 140.3 104.3) (width 0.375) (layer F.Cu) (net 13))
 (segment (start 143.65 105.61) (end 141.61 105.61) (width 0.375) (layer F.Cu) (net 13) (status 10))
 (segment (start 149.45 95.325) (end 149.975 95.85) (width 0.375) (layer F.Cu) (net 13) (status 20))
 (segment (start 148.05 95.325) (end 149.45 95.325) (width 0.375) (layer F.Cu) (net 13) (status 10))
 (segment (start 147.475 94.75) (end 148.05 95.325) (width 0.375) (layer F.Cu) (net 13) (status 20))
 (segment (start 146.4 94.45) (end 146.7 94.75) (width 0.375) (layer F.Cu) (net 13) (status 30))
 (segment (start 146.7 94.75) (end 147.475 94.75) (width 0.375) (layer F.Cu) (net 13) (status 10))
 (segment (start 147.325 96.05) (end 148.05 95.325) (width 0.375) (layer F.Cu) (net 13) (status 20))
 (segment (start 143.55 96.05) (end 147.325 96.05) (width 0.375) (layer F.Cu) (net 13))
 (segment (start 140.3 99.3) (end 143.55 96.05) (width 0.375) (layer F.Cu) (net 13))
 (segment (start 140.3 104.3) (end 140.3 99.3) (width 0.375) (layer F.Cu) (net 13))
 (segment (start 141.85 103.825) (end 143.645 103.825) (width 0.375) (layer F.Cu) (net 14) (status 30))
 (segment (start 154.35 90.34) (end 154.35 93.8) (width 0.25) (layer F.Cu) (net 1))
 (segment (start 154.35 93.8) (end 154.349998 93.800002) (width 0.25) (layer F.Cu) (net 1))
 (segment (start 156.69 88) (end 154.35 90.34) (width 0.25) (layer F.Cu) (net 1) (status 10))
 (segment (start 157.962551 110.007449) (end 154.35 113.62) (width 0.25) (layer F.Cu) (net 1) (status 20))
 (segment (start 157.962551 97.412555) (end 157.962551 110.007449) (width 0.25) (layer F.Cu) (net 1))
 (segment (start 154.35 93.800004) (end 157.962551 97.412555) (width 0.25) (layer F.Cu) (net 1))
 (segment (start 154.35 93.8) (end 154.35 93.800004) (width 0.25) (layer F.Cu) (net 1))
 (segment (start 157.462541 108.727459) (end 154.35 111.84) (width 0.25) (layer F.Cu) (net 2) (status 20))
 (segment (start 157.462541 97.619665) (end 157.462541 108.727459) (width 0.25) (layer F.Cu) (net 2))
 (segment (start 153.300001 93.457125) (end 157.462541 97.619665) (width 0.25) (layer F.Cu) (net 2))
 (segment (start 153.300001 88.849999) (end 153.300001 93.457125) (width 0.25) (layer F.Cu) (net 2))
 (segment (start 154.15 88) (end 153.300001 88.849999) (width 0.25) (layer F.Cu) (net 2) (status 10))
 (segment (start 156.962531 107.547479) (end 154.45001 110.06) (width 0.25) (layer F.Cu) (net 3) (status 20))
 (segment (start 156.962531 97.826775) (end 156.962531 107.547479) (width 0.25) (layer F.Cu) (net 3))
 (segment (start 151.61 92.474244) (end 156.962531 97.826775) (width 0.25) (layer F.Cu) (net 3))
 (segment (start 151.61 88) (end 151.61 92.474244) (width 0.25) (layer F.Cu) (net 3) (status 10))
 (segment (start 149.85 92.425) (end 149.825 92.45) (width 0.25) (layer F.Cu) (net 4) (status 30))
 (segment (start 149.825 88.755) (end 149.825 92.25) (width 0.25) (layer F.Cu) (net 4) (status 20))
 (segment (start 149.07 88) (end 149.825 88.755) (width 0.25) (layer F.Cu) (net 4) (status 10))
 (segment (start 156.46252 106.26749) (end 154.45001 108.28) (width 0.25) (layer F.Cu) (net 4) (status 20))
 (segment (start 156.46252 98.033886) (end 156.46252 106.26749) (width 0.25) (layer F.Cu) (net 4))
 (segment (start 150.678634 92.25) (end 156.46252 98.033886) (width 0.25) (layer F.Cu) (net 4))
 (segment (start 149.825 92.25) (end 150.678634 92.25) (width 0.25) (layer F.Cu) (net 4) (status 10))
 (segment (start 146.53 88) (end 146.9 88.37) (width 0.25) (layer F.Cu) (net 5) (status 30))
 (segment (start 155.962509 104.987501) (end 154.45001 106.5) (width 0.25) (layer F.Cu) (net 5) (status 20))
 (segment (start 155.962509 98.240997) (end 155.962509 104.987501) (width 0.25) (layer F.Cu) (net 5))
 (segment (start 152.521512 94.8) (end 155.962509 98.240997) (width 0.25) (layer F.Cu) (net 5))
 (segment (start 150.9 94.8) (end 152.521512 94.8) (width 0.25) (layer F.Cu) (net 5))
 (segment (start 149 92.9) (end 150.9 94.8) (width 0.25) (layer F.Cu) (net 5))
 (segment (start 149 90.47) (end 149 92.9) (width 0.25) (layer F.Cu) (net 5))
 (segment (start 146.53 88) (end 149 90.47) (width 0.25) (layer F.Cu) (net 5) (status 10))
 (segment (start 154.45001 102.94) (end 155.399998 101.990012) (width 0.375) (layer F.Cu) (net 7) (status 10))
 (segment (start 152.776002 95.85) (end 151.625 95.85) (width 0.375) (layer F.Cu) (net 7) (status 20))
 (segment (start 155.399998 98.473996) (end 152.776002 95.85) (width 0.375) (layer F.Cu) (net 7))
 (segment (start 155.399998 101.990012) (end 155.399998 98.473996) (width 0.375) (layer F.Cu) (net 7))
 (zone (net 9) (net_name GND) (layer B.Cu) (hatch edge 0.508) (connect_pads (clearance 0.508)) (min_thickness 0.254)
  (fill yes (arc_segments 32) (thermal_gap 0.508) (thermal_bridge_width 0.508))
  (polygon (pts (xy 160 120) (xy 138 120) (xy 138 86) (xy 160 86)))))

